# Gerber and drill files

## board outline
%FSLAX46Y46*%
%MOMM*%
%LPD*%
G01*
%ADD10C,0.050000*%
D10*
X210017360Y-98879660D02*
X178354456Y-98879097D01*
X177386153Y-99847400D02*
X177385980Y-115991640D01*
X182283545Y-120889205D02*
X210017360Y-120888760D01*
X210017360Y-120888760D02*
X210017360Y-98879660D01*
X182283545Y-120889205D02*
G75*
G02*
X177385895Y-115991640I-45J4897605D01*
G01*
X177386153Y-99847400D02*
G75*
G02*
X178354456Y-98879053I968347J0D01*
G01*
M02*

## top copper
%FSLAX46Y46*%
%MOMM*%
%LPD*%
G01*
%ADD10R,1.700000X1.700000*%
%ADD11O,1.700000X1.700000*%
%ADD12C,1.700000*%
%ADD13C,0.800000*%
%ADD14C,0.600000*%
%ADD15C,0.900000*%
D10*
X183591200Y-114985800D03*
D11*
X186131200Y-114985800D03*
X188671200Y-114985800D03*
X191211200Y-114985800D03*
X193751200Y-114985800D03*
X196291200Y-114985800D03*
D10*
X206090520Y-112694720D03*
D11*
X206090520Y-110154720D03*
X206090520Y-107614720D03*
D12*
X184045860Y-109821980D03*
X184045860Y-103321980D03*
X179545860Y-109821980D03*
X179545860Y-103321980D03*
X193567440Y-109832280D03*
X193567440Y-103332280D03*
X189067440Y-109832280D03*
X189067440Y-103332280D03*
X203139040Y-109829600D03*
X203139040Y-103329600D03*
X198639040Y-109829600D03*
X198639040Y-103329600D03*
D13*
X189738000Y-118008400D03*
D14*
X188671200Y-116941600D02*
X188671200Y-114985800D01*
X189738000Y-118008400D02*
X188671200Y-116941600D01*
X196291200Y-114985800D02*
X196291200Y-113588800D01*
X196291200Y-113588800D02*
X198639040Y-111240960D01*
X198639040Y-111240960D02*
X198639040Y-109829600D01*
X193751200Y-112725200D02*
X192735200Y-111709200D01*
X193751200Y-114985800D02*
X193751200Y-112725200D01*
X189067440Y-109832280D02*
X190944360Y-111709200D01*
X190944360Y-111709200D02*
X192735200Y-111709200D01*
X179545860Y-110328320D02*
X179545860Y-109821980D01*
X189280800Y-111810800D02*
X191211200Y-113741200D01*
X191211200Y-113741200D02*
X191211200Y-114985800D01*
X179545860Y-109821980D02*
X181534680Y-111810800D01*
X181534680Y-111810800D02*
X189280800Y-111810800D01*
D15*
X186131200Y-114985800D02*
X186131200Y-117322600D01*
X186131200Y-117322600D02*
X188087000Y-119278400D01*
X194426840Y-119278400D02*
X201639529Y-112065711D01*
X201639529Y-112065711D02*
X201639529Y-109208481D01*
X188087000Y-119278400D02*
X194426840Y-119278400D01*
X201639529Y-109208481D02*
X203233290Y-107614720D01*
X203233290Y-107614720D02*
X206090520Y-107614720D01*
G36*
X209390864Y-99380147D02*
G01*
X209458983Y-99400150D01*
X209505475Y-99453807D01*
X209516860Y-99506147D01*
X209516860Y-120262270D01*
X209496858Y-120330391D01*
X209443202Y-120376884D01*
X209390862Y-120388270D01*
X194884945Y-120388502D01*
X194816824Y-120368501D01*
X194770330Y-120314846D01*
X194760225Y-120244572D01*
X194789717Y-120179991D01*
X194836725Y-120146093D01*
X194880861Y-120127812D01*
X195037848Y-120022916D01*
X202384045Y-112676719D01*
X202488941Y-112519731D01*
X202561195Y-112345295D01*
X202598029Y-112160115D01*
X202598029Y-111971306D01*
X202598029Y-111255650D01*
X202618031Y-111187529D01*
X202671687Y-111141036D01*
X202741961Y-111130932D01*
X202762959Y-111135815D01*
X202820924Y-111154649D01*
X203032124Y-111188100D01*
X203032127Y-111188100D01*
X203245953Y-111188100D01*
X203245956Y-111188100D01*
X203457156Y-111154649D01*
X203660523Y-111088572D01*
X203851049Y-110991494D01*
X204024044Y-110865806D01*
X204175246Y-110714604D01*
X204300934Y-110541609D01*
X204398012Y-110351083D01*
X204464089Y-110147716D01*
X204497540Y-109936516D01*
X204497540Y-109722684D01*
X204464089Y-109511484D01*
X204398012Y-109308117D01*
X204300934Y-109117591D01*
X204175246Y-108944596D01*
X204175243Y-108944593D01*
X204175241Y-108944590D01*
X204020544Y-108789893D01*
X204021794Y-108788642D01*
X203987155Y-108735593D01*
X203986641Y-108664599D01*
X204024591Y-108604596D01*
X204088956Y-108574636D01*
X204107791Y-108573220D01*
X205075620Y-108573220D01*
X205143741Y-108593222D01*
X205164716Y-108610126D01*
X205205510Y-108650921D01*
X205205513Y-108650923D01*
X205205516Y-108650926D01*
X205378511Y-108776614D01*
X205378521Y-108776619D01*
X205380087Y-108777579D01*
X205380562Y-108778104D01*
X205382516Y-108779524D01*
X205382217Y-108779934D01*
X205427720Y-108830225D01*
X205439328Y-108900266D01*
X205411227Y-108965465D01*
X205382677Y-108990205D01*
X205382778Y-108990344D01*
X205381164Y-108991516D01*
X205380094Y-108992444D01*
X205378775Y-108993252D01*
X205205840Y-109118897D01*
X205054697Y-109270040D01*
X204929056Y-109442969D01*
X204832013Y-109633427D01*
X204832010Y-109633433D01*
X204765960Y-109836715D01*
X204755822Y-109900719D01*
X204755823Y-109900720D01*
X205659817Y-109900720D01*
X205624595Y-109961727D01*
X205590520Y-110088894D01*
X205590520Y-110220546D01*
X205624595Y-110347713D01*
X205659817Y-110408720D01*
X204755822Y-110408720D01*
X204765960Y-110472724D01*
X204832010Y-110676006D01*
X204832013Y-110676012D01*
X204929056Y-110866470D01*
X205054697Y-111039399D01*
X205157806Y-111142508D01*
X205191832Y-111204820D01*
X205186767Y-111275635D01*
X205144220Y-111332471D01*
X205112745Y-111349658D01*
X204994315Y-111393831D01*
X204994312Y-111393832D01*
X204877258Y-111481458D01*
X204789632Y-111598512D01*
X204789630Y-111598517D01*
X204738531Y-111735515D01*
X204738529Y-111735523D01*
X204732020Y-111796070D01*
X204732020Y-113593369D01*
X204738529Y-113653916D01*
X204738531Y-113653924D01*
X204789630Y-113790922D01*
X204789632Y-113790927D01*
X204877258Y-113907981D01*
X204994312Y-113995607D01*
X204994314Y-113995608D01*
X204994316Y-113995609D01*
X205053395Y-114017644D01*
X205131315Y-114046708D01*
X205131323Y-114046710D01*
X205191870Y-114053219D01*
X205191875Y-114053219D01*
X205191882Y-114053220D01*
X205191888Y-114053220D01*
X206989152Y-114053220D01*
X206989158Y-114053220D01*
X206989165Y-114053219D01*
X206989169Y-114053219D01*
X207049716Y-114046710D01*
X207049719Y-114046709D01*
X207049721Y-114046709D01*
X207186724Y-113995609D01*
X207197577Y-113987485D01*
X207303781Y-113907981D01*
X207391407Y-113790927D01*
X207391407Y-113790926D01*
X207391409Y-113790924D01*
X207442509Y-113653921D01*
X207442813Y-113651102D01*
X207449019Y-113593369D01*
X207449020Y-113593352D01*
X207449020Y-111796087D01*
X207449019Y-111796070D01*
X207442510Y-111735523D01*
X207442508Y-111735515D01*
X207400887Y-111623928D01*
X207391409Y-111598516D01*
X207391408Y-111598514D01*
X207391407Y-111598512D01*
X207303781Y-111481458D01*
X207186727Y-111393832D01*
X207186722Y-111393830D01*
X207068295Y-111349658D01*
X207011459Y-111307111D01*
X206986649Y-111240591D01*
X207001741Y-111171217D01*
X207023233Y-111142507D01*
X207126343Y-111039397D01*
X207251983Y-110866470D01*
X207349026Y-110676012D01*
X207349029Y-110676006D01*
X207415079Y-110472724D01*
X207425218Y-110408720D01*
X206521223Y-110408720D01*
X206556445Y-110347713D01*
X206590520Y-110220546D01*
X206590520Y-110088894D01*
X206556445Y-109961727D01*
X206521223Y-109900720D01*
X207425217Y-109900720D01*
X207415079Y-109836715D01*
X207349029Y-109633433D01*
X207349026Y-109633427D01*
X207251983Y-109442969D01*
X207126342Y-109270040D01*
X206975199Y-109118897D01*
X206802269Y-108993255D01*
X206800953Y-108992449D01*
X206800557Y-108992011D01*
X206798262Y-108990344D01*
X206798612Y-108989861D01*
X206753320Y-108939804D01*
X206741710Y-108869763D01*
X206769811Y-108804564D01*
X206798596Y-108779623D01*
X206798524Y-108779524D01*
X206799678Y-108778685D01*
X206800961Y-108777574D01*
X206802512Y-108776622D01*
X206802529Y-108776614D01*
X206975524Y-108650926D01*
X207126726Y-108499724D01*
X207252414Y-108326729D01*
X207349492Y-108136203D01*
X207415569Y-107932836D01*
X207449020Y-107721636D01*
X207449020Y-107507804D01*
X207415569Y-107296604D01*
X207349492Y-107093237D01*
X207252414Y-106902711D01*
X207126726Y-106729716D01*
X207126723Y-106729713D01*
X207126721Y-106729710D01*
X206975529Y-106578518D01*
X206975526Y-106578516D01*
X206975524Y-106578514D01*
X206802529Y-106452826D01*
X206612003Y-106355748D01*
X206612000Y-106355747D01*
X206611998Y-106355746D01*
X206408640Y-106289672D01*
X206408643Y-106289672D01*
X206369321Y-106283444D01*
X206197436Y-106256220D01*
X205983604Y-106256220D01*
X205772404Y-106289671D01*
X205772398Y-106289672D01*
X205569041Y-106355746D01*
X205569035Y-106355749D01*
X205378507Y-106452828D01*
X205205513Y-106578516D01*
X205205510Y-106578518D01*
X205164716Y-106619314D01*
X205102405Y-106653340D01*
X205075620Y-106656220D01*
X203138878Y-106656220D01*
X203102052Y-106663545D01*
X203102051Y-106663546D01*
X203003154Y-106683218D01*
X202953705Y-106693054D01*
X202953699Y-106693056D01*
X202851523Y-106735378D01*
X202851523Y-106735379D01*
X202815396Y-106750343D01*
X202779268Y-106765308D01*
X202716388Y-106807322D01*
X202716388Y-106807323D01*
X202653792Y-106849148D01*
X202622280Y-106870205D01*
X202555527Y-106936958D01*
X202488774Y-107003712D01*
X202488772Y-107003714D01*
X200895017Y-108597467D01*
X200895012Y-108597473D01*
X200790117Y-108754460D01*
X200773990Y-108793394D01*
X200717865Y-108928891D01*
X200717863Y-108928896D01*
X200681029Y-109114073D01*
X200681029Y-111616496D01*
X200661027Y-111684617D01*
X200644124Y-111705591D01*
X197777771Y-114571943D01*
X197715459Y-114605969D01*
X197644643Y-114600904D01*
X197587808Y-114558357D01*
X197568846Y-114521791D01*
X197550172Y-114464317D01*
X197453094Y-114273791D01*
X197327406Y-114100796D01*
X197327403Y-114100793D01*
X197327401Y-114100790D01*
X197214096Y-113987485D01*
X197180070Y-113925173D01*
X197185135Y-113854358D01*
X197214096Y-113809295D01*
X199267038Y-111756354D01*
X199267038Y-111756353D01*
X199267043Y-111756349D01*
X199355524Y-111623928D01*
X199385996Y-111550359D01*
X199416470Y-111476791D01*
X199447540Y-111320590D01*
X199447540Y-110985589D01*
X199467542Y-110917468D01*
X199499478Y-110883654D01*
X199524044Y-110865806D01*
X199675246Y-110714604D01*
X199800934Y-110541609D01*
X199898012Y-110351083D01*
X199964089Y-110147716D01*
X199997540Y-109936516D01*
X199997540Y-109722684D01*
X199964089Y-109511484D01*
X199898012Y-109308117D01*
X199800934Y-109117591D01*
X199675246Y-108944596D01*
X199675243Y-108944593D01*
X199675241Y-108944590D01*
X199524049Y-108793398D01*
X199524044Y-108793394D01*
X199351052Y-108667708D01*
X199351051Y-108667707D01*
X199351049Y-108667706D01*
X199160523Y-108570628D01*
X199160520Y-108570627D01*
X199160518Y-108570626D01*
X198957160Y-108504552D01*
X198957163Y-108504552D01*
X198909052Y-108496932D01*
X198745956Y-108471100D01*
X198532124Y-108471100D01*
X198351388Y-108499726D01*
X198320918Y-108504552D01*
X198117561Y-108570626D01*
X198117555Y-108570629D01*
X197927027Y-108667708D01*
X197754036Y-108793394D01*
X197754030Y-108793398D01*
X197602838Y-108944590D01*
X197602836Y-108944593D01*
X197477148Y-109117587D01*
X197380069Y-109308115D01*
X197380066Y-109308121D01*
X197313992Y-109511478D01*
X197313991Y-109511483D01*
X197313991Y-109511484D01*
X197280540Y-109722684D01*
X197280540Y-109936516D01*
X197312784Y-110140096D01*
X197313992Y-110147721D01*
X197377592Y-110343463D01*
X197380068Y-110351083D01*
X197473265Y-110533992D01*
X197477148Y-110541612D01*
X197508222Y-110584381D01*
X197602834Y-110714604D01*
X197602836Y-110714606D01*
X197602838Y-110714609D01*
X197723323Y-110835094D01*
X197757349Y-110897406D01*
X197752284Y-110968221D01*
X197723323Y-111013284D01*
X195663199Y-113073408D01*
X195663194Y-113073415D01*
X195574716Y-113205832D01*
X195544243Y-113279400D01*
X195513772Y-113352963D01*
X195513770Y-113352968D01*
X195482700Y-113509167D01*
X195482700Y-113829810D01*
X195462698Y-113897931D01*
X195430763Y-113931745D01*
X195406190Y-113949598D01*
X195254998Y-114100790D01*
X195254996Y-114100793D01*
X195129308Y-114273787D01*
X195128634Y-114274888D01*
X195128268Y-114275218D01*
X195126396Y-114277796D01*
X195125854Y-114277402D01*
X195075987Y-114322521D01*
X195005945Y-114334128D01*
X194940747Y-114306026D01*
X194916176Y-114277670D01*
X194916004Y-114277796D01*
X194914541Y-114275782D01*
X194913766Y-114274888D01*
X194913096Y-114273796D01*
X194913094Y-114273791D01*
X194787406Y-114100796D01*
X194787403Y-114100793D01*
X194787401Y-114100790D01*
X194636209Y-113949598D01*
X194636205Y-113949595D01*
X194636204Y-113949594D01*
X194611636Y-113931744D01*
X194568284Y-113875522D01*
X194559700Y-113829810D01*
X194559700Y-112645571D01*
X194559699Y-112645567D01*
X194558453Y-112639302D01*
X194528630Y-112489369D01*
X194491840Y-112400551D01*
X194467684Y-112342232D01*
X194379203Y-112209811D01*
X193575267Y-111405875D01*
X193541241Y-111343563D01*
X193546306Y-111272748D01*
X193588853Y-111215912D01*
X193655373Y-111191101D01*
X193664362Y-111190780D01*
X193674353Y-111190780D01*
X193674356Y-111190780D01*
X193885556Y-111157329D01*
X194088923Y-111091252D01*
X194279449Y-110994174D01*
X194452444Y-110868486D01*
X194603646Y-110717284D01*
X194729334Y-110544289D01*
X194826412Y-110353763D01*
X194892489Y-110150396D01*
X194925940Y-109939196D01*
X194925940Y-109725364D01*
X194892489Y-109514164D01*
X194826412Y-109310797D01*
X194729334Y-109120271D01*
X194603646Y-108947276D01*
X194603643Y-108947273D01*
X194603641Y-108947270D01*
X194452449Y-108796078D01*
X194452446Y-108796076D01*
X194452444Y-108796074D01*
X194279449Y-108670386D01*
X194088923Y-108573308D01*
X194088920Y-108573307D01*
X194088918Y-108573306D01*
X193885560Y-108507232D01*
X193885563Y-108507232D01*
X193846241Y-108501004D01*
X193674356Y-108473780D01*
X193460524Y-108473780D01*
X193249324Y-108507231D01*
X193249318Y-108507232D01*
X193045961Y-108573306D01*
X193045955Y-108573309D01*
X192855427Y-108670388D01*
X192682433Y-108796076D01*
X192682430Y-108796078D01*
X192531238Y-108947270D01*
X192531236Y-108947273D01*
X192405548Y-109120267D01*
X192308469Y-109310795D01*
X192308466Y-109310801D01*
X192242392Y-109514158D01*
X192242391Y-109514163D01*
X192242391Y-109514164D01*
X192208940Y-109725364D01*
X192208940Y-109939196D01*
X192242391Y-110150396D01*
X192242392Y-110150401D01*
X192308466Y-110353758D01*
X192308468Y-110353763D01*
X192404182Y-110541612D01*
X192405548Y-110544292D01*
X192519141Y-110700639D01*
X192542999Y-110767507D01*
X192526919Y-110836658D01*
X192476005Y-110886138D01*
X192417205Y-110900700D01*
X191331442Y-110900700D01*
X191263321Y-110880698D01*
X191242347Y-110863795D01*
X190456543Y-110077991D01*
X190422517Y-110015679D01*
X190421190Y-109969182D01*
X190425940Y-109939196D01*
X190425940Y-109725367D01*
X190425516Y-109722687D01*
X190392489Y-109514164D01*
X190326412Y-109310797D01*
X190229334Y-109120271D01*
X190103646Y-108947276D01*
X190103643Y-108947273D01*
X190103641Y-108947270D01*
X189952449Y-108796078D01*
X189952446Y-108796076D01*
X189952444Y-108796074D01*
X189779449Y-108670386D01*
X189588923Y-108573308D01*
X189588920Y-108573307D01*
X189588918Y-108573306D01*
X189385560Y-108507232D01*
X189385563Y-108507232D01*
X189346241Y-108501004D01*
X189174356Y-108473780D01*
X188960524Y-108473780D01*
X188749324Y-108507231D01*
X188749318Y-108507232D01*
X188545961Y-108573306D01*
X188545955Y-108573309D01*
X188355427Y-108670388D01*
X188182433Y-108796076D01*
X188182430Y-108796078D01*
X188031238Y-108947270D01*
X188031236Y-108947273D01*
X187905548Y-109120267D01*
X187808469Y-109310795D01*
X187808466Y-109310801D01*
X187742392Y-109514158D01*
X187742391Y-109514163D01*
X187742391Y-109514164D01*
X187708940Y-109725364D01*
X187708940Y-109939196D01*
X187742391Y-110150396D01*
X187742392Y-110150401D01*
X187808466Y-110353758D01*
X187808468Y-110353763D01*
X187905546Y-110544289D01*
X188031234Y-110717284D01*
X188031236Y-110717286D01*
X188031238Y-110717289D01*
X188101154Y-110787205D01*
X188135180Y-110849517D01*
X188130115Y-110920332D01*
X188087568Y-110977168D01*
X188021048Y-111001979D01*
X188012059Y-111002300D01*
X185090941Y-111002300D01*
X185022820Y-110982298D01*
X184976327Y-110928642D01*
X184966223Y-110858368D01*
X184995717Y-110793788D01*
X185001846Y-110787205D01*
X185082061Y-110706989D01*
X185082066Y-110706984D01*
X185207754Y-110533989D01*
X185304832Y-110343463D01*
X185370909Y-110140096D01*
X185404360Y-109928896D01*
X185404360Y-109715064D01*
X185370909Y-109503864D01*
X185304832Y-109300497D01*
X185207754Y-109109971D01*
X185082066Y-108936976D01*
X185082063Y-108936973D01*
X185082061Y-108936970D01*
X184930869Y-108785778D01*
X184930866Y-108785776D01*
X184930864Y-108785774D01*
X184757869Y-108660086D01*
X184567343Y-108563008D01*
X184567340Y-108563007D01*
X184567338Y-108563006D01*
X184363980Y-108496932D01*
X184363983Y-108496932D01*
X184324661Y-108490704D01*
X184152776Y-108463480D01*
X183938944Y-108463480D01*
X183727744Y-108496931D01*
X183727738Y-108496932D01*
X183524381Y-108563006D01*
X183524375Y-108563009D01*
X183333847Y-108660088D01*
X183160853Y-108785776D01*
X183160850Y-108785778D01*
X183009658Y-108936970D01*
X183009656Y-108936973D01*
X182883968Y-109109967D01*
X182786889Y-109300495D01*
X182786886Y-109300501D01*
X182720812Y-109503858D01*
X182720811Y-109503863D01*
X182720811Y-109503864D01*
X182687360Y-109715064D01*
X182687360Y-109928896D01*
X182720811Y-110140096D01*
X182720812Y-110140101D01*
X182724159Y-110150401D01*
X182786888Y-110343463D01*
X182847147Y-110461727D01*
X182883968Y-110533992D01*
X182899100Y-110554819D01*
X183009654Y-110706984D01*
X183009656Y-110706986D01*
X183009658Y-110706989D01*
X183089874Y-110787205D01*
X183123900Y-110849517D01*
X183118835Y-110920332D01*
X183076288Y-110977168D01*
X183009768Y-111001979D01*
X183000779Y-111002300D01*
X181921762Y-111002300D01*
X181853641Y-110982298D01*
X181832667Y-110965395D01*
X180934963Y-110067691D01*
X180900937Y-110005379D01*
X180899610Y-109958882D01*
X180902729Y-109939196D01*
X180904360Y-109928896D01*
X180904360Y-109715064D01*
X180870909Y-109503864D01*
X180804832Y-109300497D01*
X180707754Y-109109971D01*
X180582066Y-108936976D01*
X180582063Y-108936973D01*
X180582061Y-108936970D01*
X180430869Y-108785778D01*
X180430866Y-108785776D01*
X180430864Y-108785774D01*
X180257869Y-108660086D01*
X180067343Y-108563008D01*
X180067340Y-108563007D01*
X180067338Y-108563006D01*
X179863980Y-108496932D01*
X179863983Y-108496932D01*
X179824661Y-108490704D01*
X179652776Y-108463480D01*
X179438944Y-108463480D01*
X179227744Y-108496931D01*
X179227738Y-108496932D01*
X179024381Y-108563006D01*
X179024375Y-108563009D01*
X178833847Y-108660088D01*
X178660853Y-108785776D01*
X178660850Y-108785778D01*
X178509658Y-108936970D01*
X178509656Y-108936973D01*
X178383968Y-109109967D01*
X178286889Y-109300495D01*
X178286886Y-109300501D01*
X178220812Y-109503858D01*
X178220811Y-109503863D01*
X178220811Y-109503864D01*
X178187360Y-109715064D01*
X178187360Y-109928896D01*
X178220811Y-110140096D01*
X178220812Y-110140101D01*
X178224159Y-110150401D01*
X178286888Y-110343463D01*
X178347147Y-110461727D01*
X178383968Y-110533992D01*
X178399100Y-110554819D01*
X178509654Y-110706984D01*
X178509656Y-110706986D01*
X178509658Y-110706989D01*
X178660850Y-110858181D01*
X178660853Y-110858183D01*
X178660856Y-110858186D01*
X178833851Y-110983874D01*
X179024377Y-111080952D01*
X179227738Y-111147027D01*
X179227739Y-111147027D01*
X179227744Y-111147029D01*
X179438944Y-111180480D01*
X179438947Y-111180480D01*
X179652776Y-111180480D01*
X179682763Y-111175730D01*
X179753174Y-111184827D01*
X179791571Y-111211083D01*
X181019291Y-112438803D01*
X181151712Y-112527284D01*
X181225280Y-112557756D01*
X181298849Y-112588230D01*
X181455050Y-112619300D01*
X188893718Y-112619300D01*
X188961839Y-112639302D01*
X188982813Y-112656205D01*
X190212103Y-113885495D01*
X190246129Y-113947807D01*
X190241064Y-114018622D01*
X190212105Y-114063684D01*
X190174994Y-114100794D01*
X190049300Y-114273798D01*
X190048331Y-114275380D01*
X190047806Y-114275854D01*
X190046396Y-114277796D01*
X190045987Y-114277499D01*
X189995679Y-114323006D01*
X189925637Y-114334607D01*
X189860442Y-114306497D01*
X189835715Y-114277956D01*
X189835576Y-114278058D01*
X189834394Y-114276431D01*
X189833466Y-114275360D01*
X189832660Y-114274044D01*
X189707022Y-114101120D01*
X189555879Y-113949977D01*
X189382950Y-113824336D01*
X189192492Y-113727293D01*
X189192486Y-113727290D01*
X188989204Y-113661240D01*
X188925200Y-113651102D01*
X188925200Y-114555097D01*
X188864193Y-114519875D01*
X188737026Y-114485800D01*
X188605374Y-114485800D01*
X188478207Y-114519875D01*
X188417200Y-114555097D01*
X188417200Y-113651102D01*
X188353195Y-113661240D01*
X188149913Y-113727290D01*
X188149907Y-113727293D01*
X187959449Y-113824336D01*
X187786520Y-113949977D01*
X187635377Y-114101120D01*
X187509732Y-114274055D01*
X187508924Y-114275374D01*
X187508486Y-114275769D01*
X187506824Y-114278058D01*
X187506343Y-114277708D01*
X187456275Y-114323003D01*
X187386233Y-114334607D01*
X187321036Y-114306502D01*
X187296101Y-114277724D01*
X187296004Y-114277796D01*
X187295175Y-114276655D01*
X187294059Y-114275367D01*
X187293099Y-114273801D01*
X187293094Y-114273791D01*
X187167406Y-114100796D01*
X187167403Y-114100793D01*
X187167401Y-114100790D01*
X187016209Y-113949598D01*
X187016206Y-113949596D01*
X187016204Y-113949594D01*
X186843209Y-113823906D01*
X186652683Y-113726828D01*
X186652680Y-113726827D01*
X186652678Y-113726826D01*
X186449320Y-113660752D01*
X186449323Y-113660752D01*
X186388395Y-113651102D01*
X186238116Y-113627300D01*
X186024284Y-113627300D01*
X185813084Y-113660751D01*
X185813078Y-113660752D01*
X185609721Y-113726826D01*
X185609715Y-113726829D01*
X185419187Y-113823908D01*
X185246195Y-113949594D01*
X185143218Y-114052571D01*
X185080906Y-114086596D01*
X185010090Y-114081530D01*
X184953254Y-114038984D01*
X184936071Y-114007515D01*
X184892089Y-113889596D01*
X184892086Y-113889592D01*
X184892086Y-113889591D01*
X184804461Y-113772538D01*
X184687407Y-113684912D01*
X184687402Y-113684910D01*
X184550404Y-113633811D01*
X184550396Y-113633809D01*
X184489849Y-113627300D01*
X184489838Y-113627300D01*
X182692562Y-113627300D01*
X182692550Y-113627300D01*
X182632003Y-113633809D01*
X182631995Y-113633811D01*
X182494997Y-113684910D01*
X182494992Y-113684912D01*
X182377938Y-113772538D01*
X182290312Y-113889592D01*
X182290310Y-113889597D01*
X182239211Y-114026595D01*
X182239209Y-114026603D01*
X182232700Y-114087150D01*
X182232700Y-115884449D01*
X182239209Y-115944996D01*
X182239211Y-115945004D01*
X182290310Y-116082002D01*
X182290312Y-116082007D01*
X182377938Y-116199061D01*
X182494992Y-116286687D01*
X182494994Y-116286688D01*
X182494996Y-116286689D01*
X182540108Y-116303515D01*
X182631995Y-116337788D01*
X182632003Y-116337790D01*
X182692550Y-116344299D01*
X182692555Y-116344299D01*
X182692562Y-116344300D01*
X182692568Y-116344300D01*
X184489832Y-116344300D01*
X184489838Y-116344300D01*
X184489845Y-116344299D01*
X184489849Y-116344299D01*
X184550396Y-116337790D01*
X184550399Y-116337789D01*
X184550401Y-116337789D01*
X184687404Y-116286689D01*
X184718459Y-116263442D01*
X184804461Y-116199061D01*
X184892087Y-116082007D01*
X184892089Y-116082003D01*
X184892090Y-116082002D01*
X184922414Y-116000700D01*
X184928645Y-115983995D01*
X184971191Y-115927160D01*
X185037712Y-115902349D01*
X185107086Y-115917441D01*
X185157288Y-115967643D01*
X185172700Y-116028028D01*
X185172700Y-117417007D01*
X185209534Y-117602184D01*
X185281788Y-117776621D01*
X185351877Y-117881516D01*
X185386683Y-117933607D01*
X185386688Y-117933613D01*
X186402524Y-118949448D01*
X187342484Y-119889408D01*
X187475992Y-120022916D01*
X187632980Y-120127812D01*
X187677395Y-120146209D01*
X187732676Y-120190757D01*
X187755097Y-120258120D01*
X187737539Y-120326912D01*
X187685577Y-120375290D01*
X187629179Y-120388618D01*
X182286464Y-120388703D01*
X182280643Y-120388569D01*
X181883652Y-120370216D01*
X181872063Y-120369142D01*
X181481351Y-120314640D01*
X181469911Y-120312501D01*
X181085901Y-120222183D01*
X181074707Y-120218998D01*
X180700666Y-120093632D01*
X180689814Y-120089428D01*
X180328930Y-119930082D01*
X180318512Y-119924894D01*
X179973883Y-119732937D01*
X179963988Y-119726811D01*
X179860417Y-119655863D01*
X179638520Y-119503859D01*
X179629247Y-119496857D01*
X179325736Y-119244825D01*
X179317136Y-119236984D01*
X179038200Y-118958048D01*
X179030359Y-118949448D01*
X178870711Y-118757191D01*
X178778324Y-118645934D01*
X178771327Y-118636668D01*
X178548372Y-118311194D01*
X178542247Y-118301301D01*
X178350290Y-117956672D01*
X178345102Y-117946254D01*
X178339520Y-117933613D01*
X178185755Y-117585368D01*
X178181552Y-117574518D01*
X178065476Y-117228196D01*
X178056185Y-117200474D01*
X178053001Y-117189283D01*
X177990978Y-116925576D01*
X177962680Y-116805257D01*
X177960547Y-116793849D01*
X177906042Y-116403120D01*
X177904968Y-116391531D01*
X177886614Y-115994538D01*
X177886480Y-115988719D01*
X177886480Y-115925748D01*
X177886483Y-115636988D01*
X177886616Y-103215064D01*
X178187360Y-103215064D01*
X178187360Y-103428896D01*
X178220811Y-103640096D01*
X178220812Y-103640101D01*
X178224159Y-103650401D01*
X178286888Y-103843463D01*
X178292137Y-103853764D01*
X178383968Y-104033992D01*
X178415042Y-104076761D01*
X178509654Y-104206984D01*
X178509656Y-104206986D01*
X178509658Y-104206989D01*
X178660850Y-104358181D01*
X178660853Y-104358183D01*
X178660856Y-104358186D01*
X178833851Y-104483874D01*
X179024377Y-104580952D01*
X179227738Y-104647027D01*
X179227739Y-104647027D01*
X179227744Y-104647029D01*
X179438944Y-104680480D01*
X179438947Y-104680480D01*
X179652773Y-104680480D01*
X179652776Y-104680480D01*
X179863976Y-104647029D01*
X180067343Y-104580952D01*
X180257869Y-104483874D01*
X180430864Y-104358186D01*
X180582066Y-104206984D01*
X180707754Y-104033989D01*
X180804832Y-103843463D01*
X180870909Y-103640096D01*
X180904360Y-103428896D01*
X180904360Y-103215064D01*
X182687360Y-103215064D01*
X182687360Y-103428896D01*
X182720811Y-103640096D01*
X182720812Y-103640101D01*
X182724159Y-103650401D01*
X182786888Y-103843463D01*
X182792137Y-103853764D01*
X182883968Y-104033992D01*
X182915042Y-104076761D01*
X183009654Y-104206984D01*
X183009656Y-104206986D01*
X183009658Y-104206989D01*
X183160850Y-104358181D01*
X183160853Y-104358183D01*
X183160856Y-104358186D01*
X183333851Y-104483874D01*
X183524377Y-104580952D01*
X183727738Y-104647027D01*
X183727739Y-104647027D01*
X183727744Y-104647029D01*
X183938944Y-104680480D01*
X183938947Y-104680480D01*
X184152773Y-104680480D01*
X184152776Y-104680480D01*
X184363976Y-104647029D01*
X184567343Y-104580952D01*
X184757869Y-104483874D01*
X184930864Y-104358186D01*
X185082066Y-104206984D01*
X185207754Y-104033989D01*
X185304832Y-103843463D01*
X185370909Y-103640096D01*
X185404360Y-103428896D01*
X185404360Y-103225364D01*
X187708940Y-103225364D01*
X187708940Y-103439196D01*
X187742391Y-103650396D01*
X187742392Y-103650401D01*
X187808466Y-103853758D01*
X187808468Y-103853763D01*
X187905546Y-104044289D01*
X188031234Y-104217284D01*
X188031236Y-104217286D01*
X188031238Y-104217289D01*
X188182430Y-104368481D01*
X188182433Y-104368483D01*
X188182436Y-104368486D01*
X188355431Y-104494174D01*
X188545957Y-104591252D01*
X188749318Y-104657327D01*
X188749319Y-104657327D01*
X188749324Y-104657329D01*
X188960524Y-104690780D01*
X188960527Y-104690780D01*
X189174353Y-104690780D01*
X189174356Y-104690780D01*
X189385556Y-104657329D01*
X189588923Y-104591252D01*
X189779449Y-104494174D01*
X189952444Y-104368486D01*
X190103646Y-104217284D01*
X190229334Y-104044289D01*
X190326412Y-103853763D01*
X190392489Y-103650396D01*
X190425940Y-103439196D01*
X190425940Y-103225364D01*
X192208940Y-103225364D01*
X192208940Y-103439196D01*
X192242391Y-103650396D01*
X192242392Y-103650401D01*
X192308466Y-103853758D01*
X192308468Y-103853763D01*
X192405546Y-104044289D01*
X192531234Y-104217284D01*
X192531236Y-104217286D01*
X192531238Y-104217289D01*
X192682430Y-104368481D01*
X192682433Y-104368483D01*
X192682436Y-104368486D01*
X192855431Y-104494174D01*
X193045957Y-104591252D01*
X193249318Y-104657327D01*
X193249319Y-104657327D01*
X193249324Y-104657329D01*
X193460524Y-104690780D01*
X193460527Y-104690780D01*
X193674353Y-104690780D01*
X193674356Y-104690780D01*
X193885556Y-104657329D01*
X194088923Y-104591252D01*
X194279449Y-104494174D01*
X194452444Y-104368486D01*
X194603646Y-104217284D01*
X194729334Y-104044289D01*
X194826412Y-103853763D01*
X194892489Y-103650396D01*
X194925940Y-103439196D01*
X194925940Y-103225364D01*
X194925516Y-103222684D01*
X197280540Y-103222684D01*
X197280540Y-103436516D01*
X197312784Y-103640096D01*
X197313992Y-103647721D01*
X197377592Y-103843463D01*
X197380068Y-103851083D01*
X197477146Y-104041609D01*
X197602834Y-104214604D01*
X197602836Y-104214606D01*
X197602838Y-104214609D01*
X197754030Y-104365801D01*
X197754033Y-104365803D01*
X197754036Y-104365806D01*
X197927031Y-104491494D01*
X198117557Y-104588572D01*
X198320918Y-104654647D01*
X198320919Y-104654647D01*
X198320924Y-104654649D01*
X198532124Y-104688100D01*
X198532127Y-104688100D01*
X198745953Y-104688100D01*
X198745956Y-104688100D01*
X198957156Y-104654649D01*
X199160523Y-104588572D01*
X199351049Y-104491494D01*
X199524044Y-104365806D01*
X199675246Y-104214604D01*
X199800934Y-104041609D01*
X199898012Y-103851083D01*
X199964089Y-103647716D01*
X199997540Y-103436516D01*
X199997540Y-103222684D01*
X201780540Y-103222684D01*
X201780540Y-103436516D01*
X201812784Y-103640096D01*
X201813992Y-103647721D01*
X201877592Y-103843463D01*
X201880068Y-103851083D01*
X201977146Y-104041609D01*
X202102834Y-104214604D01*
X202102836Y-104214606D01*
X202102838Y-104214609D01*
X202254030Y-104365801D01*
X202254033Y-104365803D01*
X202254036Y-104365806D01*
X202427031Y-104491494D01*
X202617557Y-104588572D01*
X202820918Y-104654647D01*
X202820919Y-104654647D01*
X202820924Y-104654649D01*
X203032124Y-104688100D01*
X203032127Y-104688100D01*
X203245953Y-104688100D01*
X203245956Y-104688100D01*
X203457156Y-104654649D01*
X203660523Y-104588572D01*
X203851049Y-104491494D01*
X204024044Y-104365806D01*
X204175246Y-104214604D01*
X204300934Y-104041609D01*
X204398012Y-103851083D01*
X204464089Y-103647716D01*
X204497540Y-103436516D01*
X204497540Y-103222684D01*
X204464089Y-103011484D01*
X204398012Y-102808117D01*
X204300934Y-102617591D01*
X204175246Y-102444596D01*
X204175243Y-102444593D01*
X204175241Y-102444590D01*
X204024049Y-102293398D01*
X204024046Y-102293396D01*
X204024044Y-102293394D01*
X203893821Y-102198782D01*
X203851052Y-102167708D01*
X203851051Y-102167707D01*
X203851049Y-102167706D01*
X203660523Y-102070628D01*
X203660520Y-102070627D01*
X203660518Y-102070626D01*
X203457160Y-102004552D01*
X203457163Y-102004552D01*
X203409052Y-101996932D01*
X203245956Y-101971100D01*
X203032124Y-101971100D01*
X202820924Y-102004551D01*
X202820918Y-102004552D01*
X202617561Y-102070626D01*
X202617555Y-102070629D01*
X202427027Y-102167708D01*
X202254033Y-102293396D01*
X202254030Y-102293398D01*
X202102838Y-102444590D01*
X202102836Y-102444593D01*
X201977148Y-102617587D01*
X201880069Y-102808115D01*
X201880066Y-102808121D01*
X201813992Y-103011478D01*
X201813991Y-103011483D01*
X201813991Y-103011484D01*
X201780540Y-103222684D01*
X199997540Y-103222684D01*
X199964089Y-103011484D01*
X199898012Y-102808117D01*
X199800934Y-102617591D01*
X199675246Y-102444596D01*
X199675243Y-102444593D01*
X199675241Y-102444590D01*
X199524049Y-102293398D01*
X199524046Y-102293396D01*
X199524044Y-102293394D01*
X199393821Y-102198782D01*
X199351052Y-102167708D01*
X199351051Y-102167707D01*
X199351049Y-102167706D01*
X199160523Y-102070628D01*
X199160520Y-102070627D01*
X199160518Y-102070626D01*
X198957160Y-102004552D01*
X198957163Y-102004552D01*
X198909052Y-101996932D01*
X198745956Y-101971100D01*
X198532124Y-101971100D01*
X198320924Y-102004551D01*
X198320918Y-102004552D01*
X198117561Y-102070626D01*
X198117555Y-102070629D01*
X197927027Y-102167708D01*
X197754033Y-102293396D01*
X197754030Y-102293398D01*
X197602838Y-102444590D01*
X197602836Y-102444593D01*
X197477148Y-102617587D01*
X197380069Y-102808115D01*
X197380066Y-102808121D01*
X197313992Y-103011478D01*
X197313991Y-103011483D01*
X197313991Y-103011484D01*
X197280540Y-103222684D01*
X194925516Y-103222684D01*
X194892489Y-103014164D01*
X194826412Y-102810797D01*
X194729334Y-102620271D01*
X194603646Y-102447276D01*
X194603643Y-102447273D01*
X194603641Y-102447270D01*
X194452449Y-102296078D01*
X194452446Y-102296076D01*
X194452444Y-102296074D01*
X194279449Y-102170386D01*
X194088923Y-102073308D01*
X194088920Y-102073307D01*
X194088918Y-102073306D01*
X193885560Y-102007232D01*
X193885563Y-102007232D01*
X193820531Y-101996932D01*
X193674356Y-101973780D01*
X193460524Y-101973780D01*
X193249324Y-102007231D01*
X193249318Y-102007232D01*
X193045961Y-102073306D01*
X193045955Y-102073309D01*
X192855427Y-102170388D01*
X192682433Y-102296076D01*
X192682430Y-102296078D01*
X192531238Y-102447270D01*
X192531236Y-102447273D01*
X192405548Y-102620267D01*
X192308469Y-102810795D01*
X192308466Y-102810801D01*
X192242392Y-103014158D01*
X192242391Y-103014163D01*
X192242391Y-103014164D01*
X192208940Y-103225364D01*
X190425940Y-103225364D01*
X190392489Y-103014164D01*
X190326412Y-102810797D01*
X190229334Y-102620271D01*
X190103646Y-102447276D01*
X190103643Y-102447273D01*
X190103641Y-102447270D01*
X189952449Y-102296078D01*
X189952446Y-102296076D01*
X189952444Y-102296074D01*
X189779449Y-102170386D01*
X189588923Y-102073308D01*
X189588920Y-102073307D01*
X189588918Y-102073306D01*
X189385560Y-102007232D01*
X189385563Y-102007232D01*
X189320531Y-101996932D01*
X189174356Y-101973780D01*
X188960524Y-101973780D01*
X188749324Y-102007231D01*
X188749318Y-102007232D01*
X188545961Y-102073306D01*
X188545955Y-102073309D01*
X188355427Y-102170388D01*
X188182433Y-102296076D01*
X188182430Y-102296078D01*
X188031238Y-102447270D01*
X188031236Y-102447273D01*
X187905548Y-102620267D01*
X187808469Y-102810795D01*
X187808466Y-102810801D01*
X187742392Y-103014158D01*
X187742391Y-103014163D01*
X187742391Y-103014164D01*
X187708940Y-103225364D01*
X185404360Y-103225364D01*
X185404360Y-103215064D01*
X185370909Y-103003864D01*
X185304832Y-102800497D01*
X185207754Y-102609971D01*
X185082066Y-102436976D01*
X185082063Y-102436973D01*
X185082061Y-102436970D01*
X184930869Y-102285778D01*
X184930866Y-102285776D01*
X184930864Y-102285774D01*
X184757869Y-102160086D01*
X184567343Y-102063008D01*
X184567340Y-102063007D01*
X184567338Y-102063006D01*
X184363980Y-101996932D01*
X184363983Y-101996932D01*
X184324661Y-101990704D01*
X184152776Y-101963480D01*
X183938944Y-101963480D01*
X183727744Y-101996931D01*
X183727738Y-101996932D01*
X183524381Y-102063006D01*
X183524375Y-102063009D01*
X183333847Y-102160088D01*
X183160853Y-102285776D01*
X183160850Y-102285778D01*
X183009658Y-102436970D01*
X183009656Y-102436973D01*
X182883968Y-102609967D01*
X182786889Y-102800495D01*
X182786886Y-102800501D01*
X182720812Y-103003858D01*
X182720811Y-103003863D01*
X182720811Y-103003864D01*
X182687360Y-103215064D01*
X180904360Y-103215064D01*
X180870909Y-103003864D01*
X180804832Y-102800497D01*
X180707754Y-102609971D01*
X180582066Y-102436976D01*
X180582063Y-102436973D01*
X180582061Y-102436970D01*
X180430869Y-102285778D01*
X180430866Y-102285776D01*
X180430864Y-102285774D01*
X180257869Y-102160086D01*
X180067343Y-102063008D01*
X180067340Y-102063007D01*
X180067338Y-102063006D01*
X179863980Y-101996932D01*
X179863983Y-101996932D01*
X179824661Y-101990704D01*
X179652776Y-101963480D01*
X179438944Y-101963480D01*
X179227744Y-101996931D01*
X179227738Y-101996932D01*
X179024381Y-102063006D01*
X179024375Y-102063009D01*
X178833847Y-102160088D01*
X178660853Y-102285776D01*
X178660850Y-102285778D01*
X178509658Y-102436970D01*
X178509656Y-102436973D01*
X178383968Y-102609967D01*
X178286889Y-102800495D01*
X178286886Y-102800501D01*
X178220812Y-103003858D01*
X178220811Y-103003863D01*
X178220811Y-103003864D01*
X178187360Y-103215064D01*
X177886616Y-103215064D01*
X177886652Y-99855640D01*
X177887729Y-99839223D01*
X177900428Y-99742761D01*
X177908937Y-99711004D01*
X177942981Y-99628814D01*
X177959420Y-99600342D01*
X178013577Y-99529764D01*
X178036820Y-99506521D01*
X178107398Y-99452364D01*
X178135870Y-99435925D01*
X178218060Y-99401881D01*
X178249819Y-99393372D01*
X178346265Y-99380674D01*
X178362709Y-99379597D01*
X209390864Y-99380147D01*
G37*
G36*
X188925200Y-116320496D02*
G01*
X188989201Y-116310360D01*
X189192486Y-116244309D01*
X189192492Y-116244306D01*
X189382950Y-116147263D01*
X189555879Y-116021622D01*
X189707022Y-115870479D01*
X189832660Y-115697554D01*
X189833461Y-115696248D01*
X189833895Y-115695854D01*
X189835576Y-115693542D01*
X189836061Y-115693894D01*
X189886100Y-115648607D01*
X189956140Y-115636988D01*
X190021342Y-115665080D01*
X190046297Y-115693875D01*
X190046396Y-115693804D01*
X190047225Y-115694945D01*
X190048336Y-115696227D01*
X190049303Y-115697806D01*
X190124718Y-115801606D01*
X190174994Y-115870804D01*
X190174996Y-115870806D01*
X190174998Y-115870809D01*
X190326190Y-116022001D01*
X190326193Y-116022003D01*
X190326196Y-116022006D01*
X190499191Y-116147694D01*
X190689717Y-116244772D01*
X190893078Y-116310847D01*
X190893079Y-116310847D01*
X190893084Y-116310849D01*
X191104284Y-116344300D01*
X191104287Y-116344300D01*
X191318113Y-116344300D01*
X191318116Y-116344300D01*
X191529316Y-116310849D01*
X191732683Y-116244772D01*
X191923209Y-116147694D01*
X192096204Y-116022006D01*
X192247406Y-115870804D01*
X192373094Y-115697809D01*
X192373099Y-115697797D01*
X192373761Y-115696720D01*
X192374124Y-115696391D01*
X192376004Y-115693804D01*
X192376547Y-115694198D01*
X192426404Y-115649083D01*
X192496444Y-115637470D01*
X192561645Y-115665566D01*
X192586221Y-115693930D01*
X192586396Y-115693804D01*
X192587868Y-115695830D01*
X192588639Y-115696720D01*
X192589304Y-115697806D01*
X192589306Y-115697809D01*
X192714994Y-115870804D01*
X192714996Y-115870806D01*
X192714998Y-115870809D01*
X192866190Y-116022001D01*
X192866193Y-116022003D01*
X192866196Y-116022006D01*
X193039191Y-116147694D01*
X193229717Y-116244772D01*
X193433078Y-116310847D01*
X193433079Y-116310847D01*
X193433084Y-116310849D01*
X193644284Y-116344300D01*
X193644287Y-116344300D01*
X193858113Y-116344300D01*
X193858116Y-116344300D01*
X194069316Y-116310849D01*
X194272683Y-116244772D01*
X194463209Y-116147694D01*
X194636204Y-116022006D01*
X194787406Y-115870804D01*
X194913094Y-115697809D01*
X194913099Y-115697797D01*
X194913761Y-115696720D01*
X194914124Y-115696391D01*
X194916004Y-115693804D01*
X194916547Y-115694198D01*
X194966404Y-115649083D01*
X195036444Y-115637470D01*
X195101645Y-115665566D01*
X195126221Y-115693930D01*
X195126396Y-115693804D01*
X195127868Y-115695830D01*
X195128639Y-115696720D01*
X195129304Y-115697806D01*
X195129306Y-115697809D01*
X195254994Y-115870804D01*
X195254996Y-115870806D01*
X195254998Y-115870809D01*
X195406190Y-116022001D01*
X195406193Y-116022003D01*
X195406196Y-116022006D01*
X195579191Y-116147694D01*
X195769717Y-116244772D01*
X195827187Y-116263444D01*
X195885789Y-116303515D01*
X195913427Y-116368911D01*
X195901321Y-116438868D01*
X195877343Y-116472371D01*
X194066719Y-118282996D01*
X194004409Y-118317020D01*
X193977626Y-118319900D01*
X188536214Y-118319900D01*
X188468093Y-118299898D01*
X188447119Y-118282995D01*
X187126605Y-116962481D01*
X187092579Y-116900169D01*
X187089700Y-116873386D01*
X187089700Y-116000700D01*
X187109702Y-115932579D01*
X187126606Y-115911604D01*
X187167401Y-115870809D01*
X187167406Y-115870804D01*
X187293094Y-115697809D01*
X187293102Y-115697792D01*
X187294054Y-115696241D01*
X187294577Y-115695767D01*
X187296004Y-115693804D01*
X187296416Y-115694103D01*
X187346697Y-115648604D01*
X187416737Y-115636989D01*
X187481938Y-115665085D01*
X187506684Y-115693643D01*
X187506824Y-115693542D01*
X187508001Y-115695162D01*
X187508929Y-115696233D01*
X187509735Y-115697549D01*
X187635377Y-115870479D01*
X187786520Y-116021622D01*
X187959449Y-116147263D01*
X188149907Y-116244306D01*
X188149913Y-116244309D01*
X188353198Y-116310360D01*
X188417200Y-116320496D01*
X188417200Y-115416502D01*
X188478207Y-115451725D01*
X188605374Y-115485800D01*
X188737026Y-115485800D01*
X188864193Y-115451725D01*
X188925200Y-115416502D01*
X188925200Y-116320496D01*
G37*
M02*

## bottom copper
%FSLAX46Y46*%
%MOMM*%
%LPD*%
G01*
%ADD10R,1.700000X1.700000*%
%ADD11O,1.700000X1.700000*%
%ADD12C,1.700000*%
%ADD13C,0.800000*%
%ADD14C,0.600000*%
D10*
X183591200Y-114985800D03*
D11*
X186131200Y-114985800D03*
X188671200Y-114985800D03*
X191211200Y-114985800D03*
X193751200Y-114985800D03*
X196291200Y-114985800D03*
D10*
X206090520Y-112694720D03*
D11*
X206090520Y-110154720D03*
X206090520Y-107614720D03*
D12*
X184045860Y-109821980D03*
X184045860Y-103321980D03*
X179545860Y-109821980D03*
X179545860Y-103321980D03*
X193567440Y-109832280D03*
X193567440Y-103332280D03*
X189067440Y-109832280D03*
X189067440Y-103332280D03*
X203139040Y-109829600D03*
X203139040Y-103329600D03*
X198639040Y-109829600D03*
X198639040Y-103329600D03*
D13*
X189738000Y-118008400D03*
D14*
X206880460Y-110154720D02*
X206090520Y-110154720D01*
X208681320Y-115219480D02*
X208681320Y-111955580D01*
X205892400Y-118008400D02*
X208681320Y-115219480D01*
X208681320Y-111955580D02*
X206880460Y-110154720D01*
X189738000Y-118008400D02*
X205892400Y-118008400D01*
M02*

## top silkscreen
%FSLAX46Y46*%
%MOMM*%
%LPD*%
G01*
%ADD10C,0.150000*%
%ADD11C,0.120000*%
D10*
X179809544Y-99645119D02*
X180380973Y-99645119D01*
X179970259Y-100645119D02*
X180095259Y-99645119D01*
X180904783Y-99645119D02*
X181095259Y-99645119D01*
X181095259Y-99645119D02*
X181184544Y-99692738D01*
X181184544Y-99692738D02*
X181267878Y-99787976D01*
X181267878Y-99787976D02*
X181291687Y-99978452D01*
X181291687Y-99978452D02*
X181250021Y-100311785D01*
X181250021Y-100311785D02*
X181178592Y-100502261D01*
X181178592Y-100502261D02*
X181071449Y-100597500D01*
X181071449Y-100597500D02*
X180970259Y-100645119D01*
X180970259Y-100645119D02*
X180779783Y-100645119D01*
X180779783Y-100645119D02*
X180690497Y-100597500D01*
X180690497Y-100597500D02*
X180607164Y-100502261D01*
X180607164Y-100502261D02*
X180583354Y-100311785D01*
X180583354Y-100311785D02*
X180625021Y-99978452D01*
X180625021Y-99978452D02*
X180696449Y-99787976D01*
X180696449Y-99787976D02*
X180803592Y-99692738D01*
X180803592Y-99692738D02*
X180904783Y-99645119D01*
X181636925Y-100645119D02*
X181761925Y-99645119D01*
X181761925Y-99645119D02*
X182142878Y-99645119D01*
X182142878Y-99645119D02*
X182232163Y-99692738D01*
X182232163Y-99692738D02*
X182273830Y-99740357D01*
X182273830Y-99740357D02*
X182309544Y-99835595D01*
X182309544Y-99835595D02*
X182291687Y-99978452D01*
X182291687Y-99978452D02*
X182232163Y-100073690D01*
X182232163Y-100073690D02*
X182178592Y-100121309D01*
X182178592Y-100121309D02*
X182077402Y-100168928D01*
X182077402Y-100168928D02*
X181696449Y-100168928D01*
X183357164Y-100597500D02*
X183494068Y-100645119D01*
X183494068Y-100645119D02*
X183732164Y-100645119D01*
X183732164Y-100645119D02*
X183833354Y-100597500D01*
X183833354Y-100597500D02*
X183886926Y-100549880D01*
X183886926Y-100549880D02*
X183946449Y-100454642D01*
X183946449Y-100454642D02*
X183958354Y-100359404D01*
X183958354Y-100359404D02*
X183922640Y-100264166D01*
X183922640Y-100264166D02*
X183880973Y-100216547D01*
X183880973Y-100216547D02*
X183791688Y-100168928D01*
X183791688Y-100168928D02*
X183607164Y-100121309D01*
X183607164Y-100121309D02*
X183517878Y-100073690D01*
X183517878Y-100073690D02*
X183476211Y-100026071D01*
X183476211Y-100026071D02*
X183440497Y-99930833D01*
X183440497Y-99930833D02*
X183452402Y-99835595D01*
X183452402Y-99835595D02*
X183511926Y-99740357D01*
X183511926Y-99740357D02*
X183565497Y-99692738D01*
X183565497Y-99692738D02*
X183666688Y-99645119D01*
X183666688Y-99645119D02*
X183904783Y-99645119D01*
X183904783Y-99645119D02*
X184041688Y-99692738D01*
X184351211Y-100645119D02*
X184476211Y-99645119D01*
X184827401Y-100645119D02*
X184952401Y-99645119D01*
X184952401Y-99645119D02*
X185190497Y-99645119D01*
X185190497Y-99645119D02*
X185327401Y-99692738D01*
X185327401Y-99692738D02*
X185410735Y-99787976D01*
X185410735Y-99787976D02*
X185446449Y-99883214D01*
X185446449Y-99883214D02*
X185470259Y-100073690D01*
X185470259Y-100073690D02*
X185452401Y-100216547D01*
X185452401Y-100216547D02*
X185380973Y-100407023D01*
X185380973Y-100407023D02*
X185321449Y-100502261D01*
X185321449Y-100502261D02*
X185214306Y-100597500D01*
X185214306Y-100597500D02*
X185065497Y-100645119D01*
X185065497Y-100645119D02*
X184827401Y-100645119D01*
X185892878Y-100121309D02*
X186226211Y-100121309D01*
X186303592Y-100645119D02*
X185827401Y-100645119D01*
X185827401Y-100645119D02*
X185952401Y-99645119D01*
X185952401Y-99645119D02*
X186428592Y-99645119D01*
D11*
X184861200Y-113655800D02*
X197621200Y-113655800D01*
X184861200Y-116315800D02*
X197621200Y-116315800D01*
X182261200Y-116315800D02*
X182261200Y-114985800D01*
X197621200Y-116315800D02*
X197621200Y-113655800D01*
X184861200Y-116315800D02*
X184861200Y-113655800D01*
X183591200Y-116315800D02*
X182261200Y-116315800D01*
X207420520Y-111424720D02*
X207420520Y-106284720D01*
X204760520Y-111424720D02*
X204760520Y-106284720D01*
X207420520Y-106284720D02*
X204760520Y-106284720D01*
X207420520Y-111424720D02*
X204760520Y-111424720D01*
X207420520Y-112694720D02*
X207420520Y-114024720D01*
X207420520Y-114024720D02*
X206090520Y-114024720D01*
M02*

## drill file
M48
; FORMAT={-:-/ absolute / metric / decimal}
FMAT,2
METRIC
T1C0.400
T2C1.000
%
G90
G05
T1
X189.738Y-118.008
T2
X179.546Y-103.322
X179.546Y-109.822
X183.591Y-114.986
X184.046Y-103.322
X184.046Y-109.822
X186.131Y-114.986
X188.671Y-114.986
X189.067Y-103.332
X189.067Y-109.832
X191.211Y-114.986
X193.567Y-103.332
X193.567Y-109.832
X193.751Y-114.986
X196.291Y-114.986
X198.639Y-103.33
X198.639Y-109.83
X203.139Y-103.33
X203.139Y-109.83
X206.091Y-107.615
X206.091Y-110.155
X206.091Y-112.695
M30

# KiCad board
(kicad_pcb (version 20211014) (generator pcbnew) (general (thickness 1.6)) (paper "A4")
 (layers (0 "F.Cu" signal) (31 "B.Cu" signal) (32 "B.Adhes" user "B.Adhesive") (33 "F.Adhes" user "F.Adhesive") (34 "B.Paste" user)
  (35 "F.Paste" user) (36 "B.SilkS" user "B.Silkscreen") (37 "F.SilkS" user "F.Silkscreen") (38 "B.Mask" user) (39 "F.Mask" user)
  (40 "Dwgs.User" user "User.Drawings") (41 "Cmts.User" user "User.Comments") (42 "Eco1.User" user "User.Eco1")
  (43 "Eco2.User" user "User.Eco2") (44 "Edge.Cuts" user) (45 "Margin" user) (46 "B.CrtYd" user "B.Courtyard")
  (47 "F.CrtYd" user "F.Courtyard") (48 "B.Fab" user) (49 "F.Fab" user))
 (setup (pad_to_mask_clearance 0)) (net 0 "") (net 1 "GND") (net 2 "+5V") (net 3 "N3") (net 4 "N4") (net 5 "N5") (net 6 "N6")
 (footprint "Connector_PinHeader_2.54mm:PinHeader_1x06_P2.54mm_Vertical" (layer "F.Cu") (at 183.5912 114.9858 90)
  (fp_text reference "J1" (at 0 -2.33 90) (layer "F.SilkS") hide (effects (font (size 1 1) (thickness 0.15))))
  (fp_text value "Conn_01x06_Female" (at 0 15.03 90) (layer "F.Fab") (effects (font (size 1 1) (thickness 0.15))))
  (fp_line (start 1.33 1.27) (end 1.33 14.03) (layer "F.SilkS") (width 0.12))
  (fp_line (start -1.33 1.27) (end -1.33 14.03) (layer "F.SilkS") (width 0.12))
  (fp_line (start -1.33 -1.33) (end 0 -1.33) (layer "F.SilkS") (width 0.12))
  (fp_line (start -1.33 14.03) (end 1.33 14.03) (layer "F.SilkS") (width 0.12))
  (fp_line (start -1.33 1.27) (end 1.33 1.27) (layer "F.SilkS") (width 0.12))
  (fp_line (start -1.33 0) (end -1.33 -1.33) (layer "F.SilkS") (width 0.12))
  (pad "1" thru_hole rect locked (at 0 0 90) (size 1.7 1.7) (drill 1) (layers *.Cu *.Mask) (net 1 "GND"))
  (pad "2" thru_hole oval locked (at 0 2.54 90) (size 1.7 1.7) (drill 1) (layers *.Cu *.Mask) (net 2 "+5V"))
  (pad "3" thru_hole oval locked (at 0 5.08 90) (size 1.7 1.7) (drill 1) (layers *.Cu *.Mask) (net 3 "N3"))
  (pad "4" thru_hole oval locked (at 0 7.62 90) (size 1.7 1.7) (drill 1) (layers *.Cu *.Mask) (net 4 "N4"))
  (pad "5" thru_hole oval locked (at 0 10.16 90) (size 1.7 1.7) (drill 1) (layers *.Cu *.Mask) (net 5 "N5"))
  (pad "6" thru_hole oval locked (at 0 12.7 90) (size 1.7 1.7) (drill 1) (layers *.Cu *.Mask) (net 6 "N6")))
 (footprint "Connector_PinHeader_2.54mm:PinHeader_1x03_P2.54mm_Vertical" (layer "F.Cu") (at 206.09052 112.69472 180)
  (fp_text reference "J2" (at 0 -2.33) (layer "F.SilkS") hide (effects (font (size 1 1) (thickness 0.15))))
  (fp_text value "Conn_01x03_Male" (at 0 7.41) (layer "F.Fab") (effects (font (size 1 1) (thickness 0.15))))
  (fp_line (start -1.33 1.27) (end -1.33 6.41) (layer "F.SilkS") (width 0.12))
  (fp_line (start 1.33 1.27) (end 1.33 6.41) (layer "F.SilkS") (width 0.12))
  (fp_line (start -1.33 6.41) (end 1.33 6.41) (layer "F.SilkS") (width 0.12))
  (fp_line (start -1.33 1.27) (end 1.33 1.27) (layer "F.SilkS") (width 0.12))
  (fp_line (start -1.33 0) (end -1.33 -1.33) (layer "F.SilkS") (width 0.12))
  (fp_line (start -1.33 -1.33) (end 0 -1.33) (layer "F.SilkS") (width 0.12))
  (pad "1" thru_hole rect locked (at 0 0 180) (size 1.7 1.7) (drill 1) (layers *.Cu *.Mask) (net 1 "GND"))
  (pad "2" thru_hole oval locked (at 0 2.54 180) (size 1.7 1.7) (drill 1) (layers *.Cu *.Mask) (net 3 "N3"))
  (pad "3" thru_hole oval locked (at 0 5.08 180) (size 1.7 1.7) (drill 1) (layers *.Cu *.Mask) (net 2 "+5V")))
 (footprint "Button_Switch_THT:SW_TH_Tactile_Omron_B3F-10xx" (layer "B.Cu") (at 184.04586 109.82198 90)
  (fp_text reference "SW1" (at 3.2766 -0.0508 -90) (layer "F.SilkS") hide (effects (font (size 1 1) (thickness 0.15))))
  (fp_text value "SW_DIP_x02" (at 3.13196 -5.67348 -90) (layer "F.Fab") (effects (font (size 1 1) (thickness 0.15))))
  (pad "1" thru_hole circle locked (at 0 0 90) (size 1.7 1.7) (drill 1) (layers *.Cu *.Mask))
  (pad "2" thru_hole circle locked (at 6.5 0 90) (size 1.7 1.7) (drill 1) (layers *.Cu *.Mask) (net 1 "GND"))
  (pad "3" thru_hole circle locked (at 0 -4.5 90) (size 1.7 1.7) (drill 1) (layers *.Cu *.Mask) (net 4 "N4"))
  (pad "4" thru_hole circle locked (at 6.5 -4.5 90) (size 1.7 1.7) (drill 1) (layers *.Cu *.Mask)))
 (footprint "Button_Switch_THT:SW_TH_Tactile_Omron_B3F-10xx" (layer "B.Cu") (at 193.56744 109.83228 90)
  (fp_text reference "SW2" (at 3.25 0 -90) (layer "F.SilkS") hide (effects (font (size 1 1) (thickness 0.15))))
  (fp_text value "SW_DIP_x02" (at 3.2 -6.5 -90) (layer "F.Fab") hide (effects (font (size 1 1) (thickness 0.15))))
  (pad "1" thru_hole circle locked (at 0 0 90) (size 1.7 1.7) (drill 1) (layers *.Cu *.Mask))
  (pad "2" thru_hole circle locked (at 6.5 0 90) (size 1.7 1.7) (drill 1) (layers *.Cu *.Mask) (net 1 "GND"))
  (pad "3" thru_hole circle locked (at 0 -4.5 90) (size 1.7 1.7) (drill 1) (layers *.Cu *.Mask) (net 5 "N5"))
  (pad "4" thru_hole circle locked (at 6.5 -4.5 90) (size 1.7 1.7) (drill 1) (layers *.Cu *.Mask)))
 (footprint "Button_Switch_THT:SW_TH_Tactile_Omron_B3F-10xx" (layer "B.Cu") (at 203.13904 109.8296 90)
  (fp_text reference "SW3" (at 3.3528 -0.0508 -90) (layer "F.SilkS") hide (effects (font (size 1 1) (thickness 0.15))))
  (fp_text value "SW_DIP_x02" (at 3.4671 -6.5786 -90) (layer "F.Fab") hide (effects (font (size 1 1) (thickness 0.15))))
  (pad "1" thru_hole circle locked (at 0 0 90) (size 1.7 1.7) (drill 1) (layers *.Cu *.Mask))
  (pad "2" thru_hole circle locked (at 6.5 0 90) (size 1.7 1.7) (drill 1) (layers *.Cu *.Mask) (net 1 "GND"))
  (pad "3" thru_hole circle locked (at 0 -4.5 90) (size 1.7 1.7) (drill 1) (layers *.Cu *.Mask) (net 6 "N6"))
  (pad "4" thru_hole circle locked (at 6.5 -4.5 90) (size 1.7 1.7) (drill 1) (layers *.Cu *.Mask)))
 (gr_line (start 210.01736 98.87966) (end 178.354456 98.879097) (layer "Edge.Cuts") (width 0.05))
 (gr_line (start 177.386153 99.8474) (end 177.38598 115.99164) (layer "Edge.Cuts") (width 0.05))
 (gr_line (start 182.283545 120.889205) (end 210.01736 120.88876) (layer "Edge.Cuts") (width 0.05))
 (gr_line (start 210.01736 120.88876) (end 210.01736 98.87966) (layer "Edge.Cuts") (width 0.05))
 (gr_arc (start 182.283545 120.889205) (mid 178.820444 119.454741) (end 177.38598 115.99164) (layer "Edge.Cuts") (width 0.05))
 (gr_arc (start 177.386153 99.8474) (mid 177.669762 99.162706) (end 178.354456 98.879097) (layer "Edge.Cuts") (width 0.05))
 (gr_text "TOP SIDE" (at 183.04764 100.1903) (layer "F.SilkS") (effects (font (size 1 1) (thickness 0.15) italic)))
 (segment (start 188.6712 116.9416) (end 188.6712 114.9858) (width 0.6) (layer "F.Cu") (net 3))
 (segment (start 189.738 118.0084) (end 188.6712 116.9416) (width 0.6) (layer "F.Cu") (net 3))
 (via (at 189.738 118.0084) (size 0.8) (drill 0.4) (layers "F.Cu" "B.Cu") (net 3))
 (segment (start 206.88046 110.15472) (end 206.09052 110.15472) (width 0.6) (layer "B.Cu") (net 3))
 (segment (start 208.68132 115.21948) (end 208.68132 111.95558) (width 0.6) (layer "B.Cu") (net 3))
 (segment (start 205.8924 118.0084) (end 208.68132 115.21948) (width 0.6) (layer "B.Cu") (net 3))
 (segment (start 208.68132 111.95558) (end 206.88046 110.15472) (width 0.6) (layer "B.Cu") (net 3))
 (segment (start 189.738 118.0084) (end 205.8924 118.0084) (width 0.6) (layer "B.Cu") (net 3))
 (segment (start 196.2912 114.9858) (end 196.2912 113.5888) (width 0.6) (layer "F.Cu") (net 6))
 (segment (start 196.2912 113.5888) (end 198.63904 111.24096) (width 0.6) (layer "F.Cu") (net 6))
 (segment (start 198.63904 111.24096) (end 198.63904 109.8296) (width 0.6) (layer "F.Cu") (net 6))
 (segment (start 193.7512 112.7252) (end 192.7352 111.7092) (width 0.6) (layer "F.Cu") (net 5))
 (segment (start 193.7512 114.9858) (end 193.7512 112.7252) (width 0.6) (layer "F.Cu") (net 5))
 (segment (start 189.06744 109.83228) (end 190.94436 111.7092) (width 0.6) (layer "F.Cu") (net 5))
 (segment (start 190.94436 111.7092) (end 192.7352 111.7092) (width 0.6) (layer "F.Cu") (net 5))
 (segment (start 179.54586 110.32832) (end 179.54586 109.82198) (width 0.6) (layer "F.Cu") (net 4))
 (segment (start 189.2808 111.8108) (end 191.2112 113.7412) (width 0.6) (layer "F.Cu") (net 4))
 (segment (start 191.2112 113.7412) (end 191.2112 114.9858) (width 0.6) (layer "F.Cu") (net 4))
 (segment (start 179.54586 109.82198) (end 181.53468 111.8108) (width 0.6) (layer "F.Cu") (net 4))
 (segment (start 181.53468 111.8108) (end 189.2808 111.8108) (width 0.6) (layer "F.Cu") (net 4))
 (segment (start 186.1312 114.9858) (end 186.1312 117.3226) (width 0.9) (layer "F.Cu") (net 2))
 (segment (start 186.1312 117.3226) (end 188.087 119.2784) (width 0.9) (layer "F.Cu") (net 2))
 (segment (start 194.42684 119.2784) (end 201.639529 112.065711) (width 0.9) (layer "F.Cu") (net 2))
 (segment (start 201.639529 112.065711) (end 201.639529 109.208481) (width 0.9) (layer "F.Cu") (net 2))
 (segment (start 188.087 119.2784) (end 194.42684 119.2784) (width 0.9) (layer "F.Cu") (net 2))
 (segment (start 201.639529 109.208481) (end 203.23329 107.61472) (width 0.9) (layer "F.Cu") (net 2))
 (segment (start 203.23329 107.61472) (end 206.09052 107.61472) (width 0.9) (layer "F.Cu") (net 2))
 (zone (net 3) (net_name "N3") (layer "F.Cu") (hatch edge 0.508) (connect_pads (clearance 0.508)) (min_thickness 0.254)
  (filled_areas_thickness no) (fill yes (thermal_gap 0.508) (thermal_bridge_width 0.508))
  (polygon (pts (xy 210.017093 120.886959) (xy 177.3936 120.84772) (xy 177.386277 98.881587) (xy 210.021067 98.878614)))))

